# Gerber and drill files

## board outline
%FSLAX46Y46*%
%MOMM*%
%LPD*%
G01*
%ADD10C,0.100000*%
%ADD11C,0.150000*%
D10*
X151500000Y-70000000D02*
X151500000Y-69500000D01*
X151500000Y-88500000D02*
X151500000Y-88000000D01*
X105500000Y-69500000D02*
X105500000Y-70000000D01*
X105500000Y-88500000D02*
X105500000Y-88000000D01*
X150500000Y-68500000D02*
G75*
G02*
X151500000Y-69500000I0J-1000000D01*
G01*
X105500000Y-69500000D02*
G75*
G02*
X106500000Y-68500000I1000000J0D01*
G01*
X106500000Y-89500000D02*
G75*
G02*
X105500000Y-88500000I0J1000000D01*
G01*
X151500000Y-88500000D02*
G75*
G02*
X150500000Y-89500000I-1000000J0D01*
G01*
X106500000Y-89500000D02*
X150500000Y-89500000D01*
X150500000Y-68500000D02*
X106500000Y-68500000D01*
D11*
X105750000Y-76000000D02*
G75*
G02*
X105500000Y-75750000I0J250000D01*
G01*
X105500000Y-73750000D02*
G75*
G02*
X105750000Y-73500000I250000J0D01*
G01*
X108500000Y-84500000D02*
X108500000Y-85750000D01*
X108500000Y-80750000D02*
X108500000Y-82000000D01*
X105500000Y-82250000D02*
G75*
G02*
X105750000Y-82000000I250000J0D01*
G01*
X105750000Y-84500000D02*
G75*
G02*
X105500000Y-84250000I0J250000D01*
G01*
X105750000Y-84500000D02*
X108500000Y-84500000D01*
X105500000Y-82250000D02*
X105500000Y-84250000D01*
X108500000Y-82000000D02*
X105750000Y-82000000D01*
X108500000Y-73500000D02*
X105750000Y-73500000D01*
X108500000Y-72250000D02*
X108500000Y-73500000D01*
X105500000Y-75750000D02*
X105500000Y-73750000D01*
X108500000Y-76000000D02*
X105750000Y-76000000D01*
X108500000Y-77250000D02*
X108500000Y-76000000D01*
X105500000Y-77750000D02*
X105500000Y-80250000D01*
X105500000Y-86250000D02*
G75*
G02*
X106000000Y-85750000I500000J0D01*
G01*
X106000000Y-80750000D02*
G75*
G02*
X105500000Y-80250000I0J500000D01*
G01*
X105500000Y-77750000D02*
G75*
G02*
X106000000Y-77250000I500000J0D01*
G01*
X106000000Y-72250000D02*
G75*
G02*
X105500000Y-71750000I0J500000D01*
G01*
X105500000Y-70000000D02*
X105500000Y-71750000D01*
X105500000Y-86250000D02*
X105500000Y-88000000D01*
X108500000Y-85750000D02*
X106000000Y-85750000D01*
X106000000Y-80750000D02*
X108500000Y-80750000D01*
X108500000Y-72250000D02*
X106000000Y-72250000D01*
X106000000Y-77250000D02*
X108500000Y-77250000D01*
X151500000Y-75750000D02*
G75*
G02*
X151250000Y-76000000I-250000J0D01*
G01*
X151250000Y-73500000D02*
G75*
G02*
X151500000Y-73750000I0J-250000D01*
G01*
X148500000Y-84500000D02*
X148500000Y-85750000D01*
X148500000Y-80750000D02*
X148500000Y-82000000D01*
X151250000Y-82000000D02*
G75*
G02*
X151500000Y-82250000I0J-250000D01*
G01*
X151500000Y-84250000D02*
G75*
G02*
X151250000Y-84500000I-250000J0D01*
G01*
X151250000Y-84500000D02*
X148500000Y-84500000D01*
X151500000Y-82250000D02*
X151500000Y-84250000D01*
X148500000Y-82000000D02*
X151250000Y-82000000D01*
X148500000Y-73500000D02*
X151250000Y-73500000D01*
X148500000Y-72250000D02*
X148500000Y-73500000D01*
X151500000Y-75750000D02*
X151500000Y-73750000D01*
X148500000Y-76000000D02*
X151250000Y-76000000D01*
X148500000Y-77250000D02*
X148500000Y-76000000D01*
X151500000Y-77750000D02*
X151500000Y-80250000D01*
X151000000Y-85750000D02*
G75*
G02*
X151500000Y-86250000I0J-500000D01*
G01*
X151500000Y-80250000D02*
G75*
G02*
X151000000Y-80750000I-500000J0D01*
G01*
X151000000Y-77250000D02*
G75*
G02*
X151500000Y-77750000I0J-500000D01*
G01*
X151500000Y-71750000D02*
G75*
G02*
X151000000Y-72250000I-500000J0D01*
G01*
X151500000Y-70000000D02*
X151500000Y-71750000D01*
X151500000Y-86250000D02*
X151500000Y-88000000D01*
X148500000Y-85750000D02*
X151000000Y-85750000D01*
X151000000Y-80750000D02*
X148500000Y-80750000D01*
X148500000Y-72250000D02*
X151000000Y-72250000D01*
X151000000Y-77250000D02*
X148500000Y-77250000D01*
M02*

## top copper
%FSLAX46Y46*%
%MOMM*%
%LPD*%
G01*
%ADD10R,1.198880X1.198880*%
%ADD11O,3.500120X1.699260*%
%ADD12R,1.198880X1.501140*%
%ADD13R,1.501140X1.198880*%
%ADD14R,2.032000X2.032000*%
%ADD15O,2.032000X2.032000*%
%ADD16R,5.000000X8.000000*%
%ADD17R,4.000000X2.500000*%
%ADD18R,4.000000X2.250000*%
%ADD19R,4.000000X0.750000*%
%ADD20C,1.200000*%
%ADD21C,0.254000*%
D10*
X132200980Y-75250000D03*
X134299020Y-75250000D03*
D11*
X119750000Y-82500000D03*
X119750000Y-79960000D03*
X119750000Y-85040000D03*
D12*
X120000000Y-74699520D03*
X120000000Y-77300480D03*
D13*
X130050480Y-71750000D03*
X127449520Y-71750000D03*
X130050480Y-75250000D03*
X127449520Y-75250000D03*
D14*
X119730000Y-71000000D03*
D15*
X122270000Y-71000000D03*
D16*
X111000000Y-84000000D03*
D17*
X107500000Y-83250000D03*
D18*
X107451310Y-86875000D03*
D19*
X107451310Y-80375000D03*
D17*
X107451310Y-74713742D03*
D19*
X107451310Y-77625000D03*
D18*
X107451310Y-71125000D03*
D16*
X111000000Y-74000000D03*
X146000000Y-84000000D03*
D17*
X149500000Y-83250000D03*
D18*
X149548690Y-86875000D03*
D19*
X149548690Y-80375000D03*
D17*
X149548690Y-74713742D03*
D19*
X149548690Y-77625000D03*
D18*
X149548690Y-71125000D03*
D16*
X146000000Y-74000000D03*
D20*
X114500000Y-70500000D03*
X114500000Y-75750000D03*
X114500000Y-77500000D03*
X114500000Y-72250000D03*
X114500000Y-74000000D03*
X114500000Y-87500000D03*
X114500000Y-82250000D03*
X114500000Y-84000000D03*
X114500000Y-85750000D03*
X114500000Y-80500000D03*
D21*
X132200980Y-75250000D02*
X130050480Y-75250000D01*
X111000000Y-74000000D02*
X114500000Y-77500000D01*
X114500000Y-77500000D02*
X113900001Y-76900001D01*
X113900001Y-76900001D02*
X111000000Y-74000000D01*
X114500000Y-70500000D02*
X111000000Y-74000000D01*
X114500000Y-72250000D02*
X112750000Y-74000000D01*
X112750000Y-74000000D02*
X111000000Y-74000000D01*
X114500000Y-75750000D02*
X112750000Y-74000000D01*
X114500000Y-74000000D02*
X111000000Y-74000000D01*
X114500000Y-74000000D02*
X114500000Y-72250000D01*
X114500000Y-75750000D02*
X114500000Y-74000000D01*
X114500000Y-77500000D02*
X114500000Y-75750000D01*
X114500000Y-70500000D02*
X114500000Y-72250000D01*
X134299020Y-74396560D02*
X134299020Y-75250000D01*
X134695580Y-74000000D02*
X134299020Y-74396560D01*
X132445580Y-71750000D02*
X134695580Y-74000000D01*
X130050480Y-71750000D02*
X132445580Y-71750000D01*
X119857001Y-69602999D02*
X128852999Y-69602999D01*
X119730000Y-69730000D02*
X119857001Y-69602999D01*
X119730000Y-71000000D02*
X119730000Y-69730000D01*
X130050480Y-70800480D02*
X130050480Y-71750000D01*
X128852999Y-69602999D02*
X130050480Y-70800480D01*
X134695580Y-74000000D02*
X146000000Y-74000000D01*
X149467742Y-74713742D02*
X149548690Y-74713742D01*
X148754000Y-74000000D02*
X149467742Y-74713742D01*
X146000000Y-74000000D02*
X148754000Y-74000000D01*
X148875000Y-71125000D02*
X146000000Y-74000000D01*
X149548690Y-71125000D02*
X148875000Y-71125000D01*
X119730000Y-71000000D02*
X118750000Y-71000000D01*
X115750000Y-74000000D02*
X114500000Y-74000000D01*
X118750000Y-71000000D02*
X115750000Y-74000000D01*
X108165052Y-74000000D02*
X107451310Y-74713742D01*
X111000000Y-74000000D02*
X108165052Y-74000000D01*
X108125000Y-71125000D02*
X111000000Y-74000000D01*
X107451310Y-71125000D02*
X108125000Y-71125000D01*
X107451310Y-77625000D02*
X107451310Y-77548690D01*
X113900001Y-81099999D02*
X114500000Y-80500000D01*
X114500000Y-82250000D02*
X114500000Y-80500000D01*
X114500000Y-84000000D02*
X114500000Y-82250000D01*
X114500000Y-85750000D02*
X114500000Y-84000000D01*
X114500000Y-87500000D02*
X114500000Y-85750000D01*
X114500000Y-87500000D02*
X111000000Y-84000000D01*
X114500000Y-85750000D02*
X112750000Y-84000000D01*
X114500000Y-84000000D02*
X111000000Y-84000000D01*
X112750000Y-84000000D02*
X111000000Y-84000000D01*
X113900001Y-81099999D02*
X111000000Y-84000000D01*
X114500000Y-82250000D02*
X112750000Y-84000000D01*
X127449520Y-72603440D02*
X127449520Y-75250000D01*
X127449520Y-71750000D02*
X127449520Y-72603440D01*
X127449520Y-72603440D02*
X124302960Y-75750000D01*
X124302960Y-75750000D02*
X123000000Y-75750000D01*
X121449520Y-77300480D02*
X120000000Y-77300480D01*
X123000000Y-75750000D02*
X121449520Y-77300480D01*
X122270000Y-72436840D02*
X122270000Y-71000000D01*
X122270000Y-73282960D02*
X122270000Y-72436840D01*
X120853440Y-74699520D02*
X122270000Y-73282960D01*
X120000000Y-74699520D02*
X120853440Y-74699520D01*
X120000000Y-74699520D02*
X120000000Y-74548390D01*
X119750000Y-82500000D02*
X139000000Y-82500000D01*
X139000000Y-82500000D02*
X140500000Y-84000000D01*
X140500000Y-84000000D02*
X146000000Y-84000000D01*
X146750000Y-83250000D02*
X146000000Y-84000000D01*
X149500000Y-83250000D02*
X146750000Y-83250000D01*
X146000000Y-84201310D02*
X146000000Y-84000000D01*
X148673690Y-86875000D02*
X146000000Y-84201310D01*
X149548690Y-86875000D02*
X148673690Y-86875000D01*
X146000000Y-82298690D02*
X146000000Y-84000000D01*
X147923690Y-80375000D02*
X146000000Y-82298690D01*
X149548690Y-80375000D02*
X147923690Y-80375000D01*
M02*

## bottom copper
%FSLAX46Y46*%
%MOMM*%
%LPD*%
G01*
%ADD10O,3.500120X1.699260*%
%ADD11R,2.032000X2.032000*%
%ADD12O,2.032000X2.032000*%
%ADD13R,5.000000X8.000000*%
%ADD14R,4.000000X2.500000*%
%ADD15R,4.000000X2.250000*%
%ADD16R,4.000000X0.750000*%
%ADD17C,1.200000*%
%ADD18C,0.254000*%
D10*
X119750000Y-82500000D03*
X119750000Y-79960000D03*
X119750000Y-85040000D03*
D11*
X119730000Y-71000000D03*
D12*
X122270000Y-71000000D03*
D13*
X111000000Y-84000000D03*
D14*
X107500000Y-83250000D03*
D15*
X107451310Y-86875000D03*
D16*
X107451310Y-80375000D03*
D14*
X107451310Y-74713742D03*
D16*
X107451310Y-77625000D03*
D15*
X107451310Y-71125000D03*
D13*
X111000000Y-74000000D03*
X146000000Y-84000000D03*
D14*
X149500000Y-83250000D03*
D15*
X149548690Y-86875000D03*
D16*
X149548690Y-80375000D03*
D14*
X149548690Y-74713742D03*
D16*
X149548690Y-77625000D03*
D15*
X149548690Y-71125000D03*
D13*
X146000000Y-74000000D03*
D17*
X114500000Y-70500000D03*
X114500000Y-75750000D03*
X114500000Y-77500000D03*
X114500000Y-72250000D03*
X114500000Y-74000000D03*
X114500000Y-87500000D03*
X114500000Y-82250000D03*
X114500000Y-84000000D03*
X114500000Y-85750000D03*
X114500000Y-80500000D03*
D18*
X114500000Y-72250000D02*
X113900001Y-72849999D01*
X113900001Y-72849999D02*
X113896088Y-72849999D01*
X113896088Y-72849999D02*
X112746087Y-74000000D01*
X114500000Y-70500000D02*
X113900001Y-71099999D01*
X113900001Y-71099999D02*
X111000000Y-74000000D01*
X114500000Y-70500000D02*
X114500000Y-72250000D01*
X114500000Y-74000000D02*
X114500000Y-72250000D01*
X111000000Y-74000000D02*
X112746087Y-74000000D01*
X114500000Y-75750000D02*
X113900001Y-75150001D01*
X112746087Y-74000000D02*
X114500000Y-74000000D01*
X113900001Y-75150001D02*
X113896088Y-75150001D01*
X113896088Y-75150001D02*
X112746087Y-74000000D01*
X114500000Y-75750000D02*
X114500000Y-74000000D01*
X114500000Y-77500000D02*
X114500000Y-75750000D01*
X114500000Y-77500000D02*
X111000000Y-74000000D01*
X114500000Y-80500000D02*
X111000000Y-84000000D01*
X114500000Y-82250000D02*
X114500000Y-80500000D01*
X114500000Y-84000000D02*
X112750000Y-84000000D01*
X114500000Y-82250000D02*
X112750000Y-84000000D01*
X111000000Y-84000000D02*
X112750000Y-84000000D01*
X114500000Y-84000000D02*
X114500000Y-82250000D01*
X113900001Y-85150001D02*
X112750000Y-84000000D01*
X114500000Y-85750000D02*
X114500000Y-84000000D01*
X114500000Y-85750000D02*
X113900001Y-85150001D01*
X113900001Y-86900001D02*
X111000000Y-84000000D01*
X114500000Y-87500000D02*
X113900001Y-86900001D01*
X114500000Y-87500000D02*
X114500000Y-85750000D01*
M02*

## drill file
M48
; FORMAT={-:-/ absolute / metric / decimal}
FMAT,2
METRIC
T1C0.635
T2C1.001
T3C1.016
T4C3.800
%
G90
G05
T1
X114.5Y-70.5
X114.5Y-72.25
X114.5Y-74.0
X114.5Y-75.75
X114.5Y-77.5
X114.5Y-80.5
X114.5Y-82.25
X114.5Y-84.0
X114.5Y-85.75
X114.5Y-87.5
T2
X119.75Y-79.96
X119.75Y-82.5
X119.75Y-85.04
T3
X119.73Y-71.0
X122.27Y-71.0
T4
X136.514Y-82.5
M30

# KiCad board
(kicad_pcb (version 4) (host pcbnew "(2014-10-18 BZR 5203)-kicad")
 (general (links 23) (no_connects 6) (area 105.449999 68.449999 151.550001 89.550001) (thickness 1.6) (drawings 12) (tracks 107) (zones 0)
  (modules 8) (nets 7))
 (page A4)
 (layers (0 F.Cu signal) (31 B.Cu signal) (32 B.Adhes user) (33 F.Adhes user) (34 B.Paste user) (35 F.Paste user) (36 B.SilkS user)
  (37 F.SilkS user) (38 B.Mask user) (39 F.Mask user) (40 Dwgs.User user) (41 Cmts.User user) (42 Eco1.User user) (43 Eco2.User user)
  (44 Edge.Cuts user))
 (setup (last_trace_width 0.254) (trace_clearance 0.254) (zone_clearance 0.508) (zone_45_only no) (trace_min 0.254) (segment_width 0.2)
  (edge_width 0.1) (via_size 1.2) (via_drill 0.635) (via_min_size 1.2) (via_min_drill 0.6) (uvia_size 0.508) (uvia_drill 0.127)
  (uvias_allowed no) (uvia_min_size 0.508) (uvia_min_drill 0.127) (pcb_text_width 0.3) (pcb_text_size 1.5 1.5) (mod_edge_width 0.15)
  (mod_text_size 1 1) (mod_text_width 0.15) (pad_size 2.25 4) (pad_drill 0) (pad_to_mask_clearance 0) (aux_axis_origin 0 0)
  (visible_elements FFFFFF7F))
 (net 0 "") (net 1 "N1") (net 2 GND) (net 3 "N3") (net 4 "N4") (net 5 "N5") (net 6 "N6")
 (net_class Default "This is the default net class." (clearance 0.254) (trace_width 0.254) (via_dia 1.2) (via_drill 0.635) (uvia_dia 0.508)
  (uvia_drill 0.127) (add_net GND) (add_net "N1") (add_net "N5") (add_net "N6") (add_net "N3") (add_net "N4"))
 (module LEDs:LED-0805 (layer F.Cu) (at 133.25 75.25)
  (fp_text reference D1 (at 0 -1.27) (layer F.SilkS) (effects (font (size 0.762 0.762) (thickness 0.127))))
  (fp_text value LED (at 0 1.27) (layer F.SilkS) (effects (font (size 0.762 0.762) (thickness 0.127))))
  (pad 1 smd rect (at -1.04902 0) (size 1.19888 1.19888) (layers F.Cu F.Paste F.Mask) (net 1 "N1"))
  (pad 2 smd rect (at 1.04902 0) (size 1.19888 1.19888) (layers F.Cu F.Paste F.Mask) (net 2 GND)))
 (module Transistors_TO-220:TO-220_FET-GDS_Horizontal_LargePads (layer F.Cu) (at 119.75 82.5 270)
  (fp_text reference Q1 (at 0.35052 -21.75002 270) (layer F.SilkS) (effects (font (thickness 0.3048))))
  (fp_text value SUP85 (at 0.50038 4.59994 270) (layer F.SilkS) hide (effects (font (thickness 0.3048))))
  (pad D thru_hole oval (at 0 0) (size 3.50012 1.69926) (drill 1.00076) (layers *.Cu *.Mask F.SilkS) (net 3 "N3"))
  (pad G thru_hole oval (at -2.54 0) (size 3.50012 1.69926) (drill 1.00076) (layers *.Cu *.Mask F.SilkS) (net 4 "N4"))
  (pad S thru_hole oval (at 2.54 0) (size 3.50012 1.69926) (drill 1.00076) (layers *.Cu *.Mask F.SilkS) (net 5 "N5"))
  (pad "" np_thru_hole circle (at 0 -16.764) (size 3.79984 3.79984) (drill 3.79984) (layers *.Cu *.Mask F.SilkS)))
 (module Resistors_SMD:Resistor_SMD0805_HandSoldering (layer F.Cu) (at 120 76 270)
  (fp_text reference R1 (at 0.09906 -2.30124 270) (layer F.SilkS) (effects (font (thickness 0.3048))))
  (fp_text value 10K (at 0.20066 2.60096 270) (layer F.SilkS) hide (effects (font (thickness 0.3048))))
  (pad 1 smd rect (at -1.30048 0 270) (size 1.50114 1.19888) (layers F.Cu F.Paste F.Mask) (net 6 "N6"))
  (pad 2 smd rect (at 1.30048 0 270) (size 1.50114 1.19888) (layers F.Cu F.Paste F.Mask) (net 4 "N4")))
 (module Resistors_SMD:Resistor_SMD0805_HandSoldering (layer F.Cu) (at 128.75 71.75 180)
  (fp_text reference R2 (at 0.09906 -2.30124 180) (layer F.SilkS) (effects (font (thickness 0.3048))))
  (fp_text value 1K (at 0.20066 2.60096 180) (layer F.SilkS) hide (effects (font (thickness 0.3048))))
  (pad 1 smd rect (at -1.30048 0 180) (size 1.50114 1.19888) (layers F.Cu F.Paste F.Mask) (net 2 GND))
  (pad 2 smd rect (at 1.30048 0 180) (size 1.50114 1.19888) (layers F.Cu F.Paste F.Mask) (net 4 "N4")))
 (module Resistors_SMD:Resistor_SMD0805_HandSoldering (layer F.Cu) (at 128.75 75.25 180)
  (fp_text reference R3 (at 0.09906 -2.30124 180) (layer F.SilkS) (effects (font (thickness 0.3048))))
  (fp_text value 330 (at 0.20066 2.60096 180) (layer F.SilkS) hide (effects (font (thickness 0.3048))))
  (pad 1 smd rect (at -1.30048 0 180) (size 1.50114 1.19888) (layers F.Cu F.Paste F.Mask) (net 1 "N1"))
  (pad 2 smd rect (at 1.30048 0 180) (size 1.50114 1.19888) (layers F.Cu F.Paste F.Mask) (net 4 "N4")))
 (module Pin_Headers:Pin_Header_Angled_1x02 (layer F.Cu) (at 121 71)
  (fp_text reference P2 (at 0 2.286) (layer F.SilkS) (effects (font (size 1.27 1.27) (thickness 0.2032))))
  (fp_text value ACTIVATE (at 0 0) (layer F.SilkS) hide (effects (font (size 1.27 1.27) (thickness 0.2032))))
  (pad 1 thru_hole rect (at -1.27 0) (size 2.032 2.032) (drill 1.016) (layers *.Cu *.Mask F.SilkS) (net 2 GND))
  (pad 2 thru_hole oval (at 1.27 0) (size 2.032 2.032) (drill 1.016) (layers *.Cu *.Mask F.SilkS) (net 6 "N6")))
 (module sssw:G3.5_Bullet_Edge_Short (layer B.Cu) (at 106 79 270)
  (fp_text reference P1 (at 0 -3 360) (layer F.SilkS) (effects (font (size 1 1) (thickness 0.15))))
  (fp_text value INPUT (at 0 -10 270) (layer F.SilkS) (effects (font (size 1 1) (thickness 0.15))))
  (fp_arc (start -3.25 0.25) (end -3.25 0.5) (angle -90) (layer Edge.Cuts) (width 0.15))
  (fp_arc (start -5.25 0.25) (end -5.5 0.25) (angle -90) (layer Edge.Cuts) (width 0.15))
  (fp_line (start 5.5 -2.5) (end 6.75 -2.5) (layer Edge.Cuts) (width 0.15))
  (fp_line (start 1.75 -2.5) (end 3 -2.5) (layer Edge.Cuts) (width 0.15))
  (fp_arc (start 3.25 0.25) (end 3 0.25) (angle -90) (layer Edge.Cuts) (width 0.15))
  (fp_arc (start 5.25 0.25) (end 5.25 0.5) (angle -90) (layer Edge.Cuts) (width 0.15))
  (fp_line (start 5.5 0.25) (end 5.5 -2.5) (layer Edge.Cuts) (width 0.15))
  (fp_line (start 3.25 0.5) (end 5.25 0.5) (layer Edge.Cuts) (width 0.15))
  (fp_line (start 3 -2.5) (end 3 0.25) (layer Edge.Cuts) (width 0.15))
  (fp_line (start -5.5 -2.5) (end -5.5 0.25) (layer Edge.Cuts) (width 0.15))
  (fp_line (start -6.75 -2.5) (end -5.5 -2.5) (layer Edge.Cuts) (width 0.15))
  (fp_line (start -3.25 0.5) (end -5.25 0.5) (layer Edge.Cuts) (width 0.15))
  (fp_line (start -3 -2.5) (end -3 0.25) (layer Edge.Cuts) (width 0.15))
  (fp_line (start -1.75 -2.5) (end -3 -2.5) (layer Edge.Cuts) (width 0.15))
  (fp_line (start -1.25 0.5) (end 1.25 0.5) (layer Edge.Cuts) (width 0.15))
  (fp_arc (start 7.25 0) (end 6.75 0) (angle -90) (layer Edge.Cuts) (width 0.15))
  (fp_arc (start 1.25 0) (end 1.25 0.5) (angle -90) (layer Edge.Cuts) (width 0.15))
  (fp_arc (start -1.25 0) (end -1.75 0) (angle -90) (layer Edge.Cuts) (width 0.15))
  (fp_arc (start -7.25 0) (end -7.25 0.5) (angle -90) (layer Edge.Cuts) (width 0.15))
  (fp_line (start -9 0.5) (end -7.25 0.5) (layer Edge.Cuts) (width 0.15))
  (fp_line (start 7.25 0.5) (end 9 0.5) (layer Edge.Cuts) (width 0.15))
  (fp_line (start 6.75 -2.5) (end 6.75 0) (layer Edge.Cuts) (width 0.15))
  (fp_line (start 1.75 0) (end 1.75 -2.5) (layer Edge.Cuts) (width 0.15))
  (fp_line (start -6.75 -2.5) (end -6.75 0) (layer Edge.Cuts) (width 0.15))
  (fp_line (start -1.75 0) (end -1.75 -2.5) (layer Edge.Cuts) (width 0.15))
  (pad 2 connect rect (at 5 -5 270) (size 8 5) (layers *.Cu *.Mask) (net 5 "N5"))
  (pad 2 smd rect (at 4.25 -1.5 270) (size 2.5 4) (layers *.Cu *.Mask) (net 5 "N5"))
  (pad 2 smd rect (at 7.875 -1.45131 270) (size 2.25 4) (layers *.Cu *.Mask) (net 5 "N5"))
  (pad 2 smd rect (at 1.375 -1.45131 270) (size 0.75 4) (layers *.Cu *.Mask) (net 5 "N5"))
  (pad 1 smd rect (at -4.286258 -1.45131 90) (size 2.5 4) (layers *.Cu *.Mask) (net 2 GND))
  (pad 1 smd rect (at -1.375 -1.45131 90) (size 0.75 4) (layers *.Cu *.Mask) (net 2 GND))
  (pad 1 smd rect (at -7.875 -1.45131 90) (size 2.25 4) (layers *.Cu *.Mask) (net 2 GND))
  (pad 1 connect rect (at -5 -5 90) (size 8 5) (layers *.Cu *.Mask) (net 2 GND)))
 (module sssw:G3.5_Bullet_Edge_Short (layer F.Cu) (at 151 79 270)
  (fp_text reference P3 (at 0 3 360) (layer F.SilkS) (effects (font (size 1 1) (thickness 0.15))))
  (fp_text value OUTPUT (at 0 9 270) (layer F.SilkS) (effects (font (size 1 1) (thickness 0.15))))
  (fp_arc (start -3.25 -0.25) (end -3.25 -0.5) (angle 90) (layer Edge.Cuts) (width 0.15))
  (fp_arc (start -5.25 -0.25) (end -5.5 -0.25) (angle 90) (layer Edge.Cuts) (width 0.15))
  (fp_line (start 5.5 2.5) (end 6.75 2.5) (layer Edge.Cuts) (width 0.15))
  (fp_line (start 1.75 2.5) (end 3 2.5) (layer Edge.Cuts) (width 0.15))
  (fp_arc (start 3.25 -0.25) (end 3 -0.25) (angle 90) (layer Edge.Cuts) (width 0.15))
  (fp_arc (start 5.25 -0.25) (end 5.25 -0.5) (angle 90) (layer Edge.Cuts) (width 0.15))
  (fp_line (start 5.5 -0.25) (end 5.5 2.5) (layer Edge.Cuts) (width 0.15))
  (fp_line (start 3.25 -0.5) (end 5.25 -0.5) (layer Edge.Cuts) (width 0.15))
  (fp_line (start 3 2.5) (end 3 -0.25) (layer Edge.Cuts) (width 0.15))
  (fp_line (start -5.5 2.5) (end -5.5 -0.25) (layer Edge.Cuts) (width 0.15))
  (fp_line (start -6.75 2.5) (end -5.5 2.5) (layer Edge.Cuts) (width 0.15))
  (fp_line (start -3.25 -0.5) (end -5.25 -0.5) (layer Edge.Cuts) (width 0.15))
  (fp_line (start -3 2.5) (end -3 -0.25) (layer Edge.Cuts) (width 0.15))
  (fp_line (start -1.75 2.5) (end -3 2.5) (layer Edge.Cuts) (width 0.15))
  (fp_line (start -1.25 -0.5) (end 1.25 -0.5) (layer Edge.Cuts) (width 0.15))
  (fp_arc (start 7.25 0) (end 6.75 0) (angle 90) (layer Edge.Cuts) (width 0.15))
  (fp_arc (start 1.25 0) (end 1.25 -0.5) (angle 90) (layer Edge.Cuts) (width 0.15))
  (fp_arc (start -1.25 0) (end -1.75 0) (angle 90) (layer Edge.Cuts) (width 0.15))
  (fp_arc (start -7.25 0) (end -7.25 -0.5) (angle 90) (layer Edge.Cuts) (width 0.15))
  (fp_line (start -9 -0.5) (end -7.25 -0.5) (layer Edge.Cuts) (width 0.15))
  (fp_line (start 7.25 -0.5) (end 9 -0.5) (layer Edge.Cuts) (width 0.15))
  (fp_line (start 6.75 2.5) (end 6.75 0) (layer Edge.Cuts) (width 0.15))
  (fp_line (start 1.75 0) (end 1.75 2.5) (layer Edge.Cuts) (width 0.15))
  (fp_line (start -6.75 2.5) (end -6.75 0) (layer Edge.Cuts) (width 0.15))
  (fp_line (start -1.75 0) (end -1.75 2.5) (layer Edge.Cuts) (width 0.15))
  (pad 2 connect rect (at 5 5 270) (size 8 5) (layers *.Cu *.Mask) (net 3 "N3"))
  (pad 2 smd rect (at 4.25 1.5 270) (size 2.5 4) (layers *.Cu *.Mask) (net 3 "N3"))
  (pad 2 smd rect (at 7.875 1.45131 270) (size 2.25 4) (layers *.Cu *.Mask) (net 3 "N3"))
  (pad 2 smd rect (at 1.375 1.45131 270) (size 0.75 4) (layers *.Cu *.Mask) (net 3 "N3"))
  (pad 1 smd rect (at -4.286258 1.45131 90) (size 2.5 4) (layers *.Cu *.Mask) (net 2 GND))
  (pad 1 smd rect (at -1.375 1.45131 90) (size 0.75 4) (layers *.Cu *.Mask) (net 2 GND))
  (pad 1 smd rect (at -7.875 1.45131 90) (size 2.25 4) (layers *.Cu *.Mask) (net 2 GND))
  (pad 1 connect rect (at -5 5 90) (size 8 5) (layers *.Cu *.Mask) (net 2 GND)))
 (gr_line (start 151.5 70) (end 151.5 69.5) (layer Edge.Cuts) (width 0.1))
 (gr_line (start 151.5 88.5) (end 151.5 88) (layer Edge.Cuts) (width 0.1))
 (gr_line (start 105.5 69.5) (end 105.5 70) (layer Edge.Cuts) (width 0.1))
 (gr_line (start 105.5 88.5) (end 105.5 88) (layer Edge.Cuts) (width 0.1))
 (gr_arc (start 150.5 69.5) (end 151.5 69.5) (angle -90) (layer Edge.Cuts) (width 0.1))
 (gr_arc (start 106.5 69.5) (end 106.5 68.5) (angle -90) (layer Edge.Cuts) (width 0.1))
 (gr_arc (start 106.5 88.5) (end 105.5 88.5) (angle -90) (layer Edge.Cuts) (width 0.1))
 (gr_arc (start 150.5 88.5) (end 151.5 88.5) (angle 90) (layer Edge.Cuts) (width 0.1))
 (gr_line (start 106.5 89.5) (end 150.5 89.5) (layer Edge.Cuts) (width 0.1))
 (gr_line (start 150.5 68.5) (end 106.5 68.5) (layer Edge.Cuts) (width 0.1))
 (segment (start 119.75 79.96) (end 119.75 80) (width 0.254) (layer Edge.Cuts) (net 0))
 (segment (start 132.20098 75.25) (end 130.05048 75.25) (width 0.254) (layer F.Cu) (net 1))
 (segment (start 114.5 72.25) (end 113.900001 72.849999) (width 0.254) (layer B.Cu) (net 2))
 (segment (start 113.900001 72.849999) (end 113.896088 72.849999) (width 0.254) (layer B.Cu) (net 2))
 (segment (start 113.896088 72.849999) (end 112.746087 74) (width 0.254) (layer B.Cu) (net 2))
 (segment (start 114.5 70.5) (end 113.900001 71.099999) (width 0.254) (layer B.Cu) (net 2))
 (segment (start 113.900001 71.099999) (end 111 74) (width 0.254) (layer B.Cu) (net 2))
 (segment (start 114.5 70.5) (end 114.5 72.25) (width 0.254) (layer B.Cu) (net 2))
 (segment (start 114.5 74) (end 114.5 72.25) (width 0.254) (layer B.Cu) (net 2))
 (segment (start 111 74) (end 112.746087 74) (width 0.254) (layer B.Cu) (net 2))
 (segment (start 114.5 75.75) (end 113.900001 75.150001) (width 0.254) (layer B.Cu) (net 2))
 (segment (start 112.746087 74) (end 114.5 74) (width 0.254) (layer B.Cu) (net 2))
 (segment (start 113.900001 75.150001) (end 113.896088 75.150001) (width 0.254) (layer B.Cu) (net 2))
 (segment (start 113.896088 75.150001) (end 112.746087 74) (width 0.254) (layer B.Cu) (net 2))
 (segment (start 114.5 75.75) (end 114.5 74) (width 0.254) (layer B.Cu) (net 2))
 (segment (start 114.5 77.5) (end 114.5 75.75) (width 0.254) (layer B.Cu) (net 2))
 (segment (start 114.5 77.5) (end 111 74) (width 0.254) (layer B.Cu) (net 2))
 (segment (start 111 74) (end 114.5 77.5) (width 0.254) (layer F.Cu) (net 2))
 (segment (start 114.5 77.5) (end 113.900001 76.900001) (width 0.254) (layer F.Cu) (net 2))
 (segment (start 113.900001 76.900001) (end 111 74) (width 0.254) (layer F.Cu) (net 2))
 (segment (start 114.5 70.5) (end 111 74) (width 0.254) (layer F.Cu) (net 2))
 (segment (start 114.5 72.25) (end 112.75 74) (width 0.254) (layer F.Cu) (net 2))
 (segment (start 112.75 74) (end 111 74) (width 0.254) (layer F.Cu) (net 2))
 (segment (start 114.5 75.75) (end 112.75 74) (width 0.254) (layer F.Cu) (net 2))
 (segment (start 114.5 74) (end 111 74) (width 0.254) (layer F.Cu) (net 2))
 (segment (start 114.5 74) (end 114.5 72.25) (width 0.254) (layer F.Cu) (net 2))
 (segment (start 114.5 75.75) (end 114.5 74) (width 0.254) (layer F.Cu) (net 2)) (via (at 114.5 70.5) (size 1.2) (layers F.Cu B.Cu) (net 2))
 (via (at 114.5 75.75) (size 1.2) (layers F.Cu B.Cu) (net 2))
 (segment (start 114.5 77.5) (end 114.5 75.75) (width 0.254) (layer F.Cu) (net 2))
 (via (at 114.5 77.5) (size 1.2) (layers F.Cu B.Cu) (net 2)) (via (at 114.5 72.25) (size 1.2) (layers F.Cu B.Cu) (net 2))
 (segment (start 114.5 70.5) (end 114.5 72.25) (width 0.254) (layer F.Cu) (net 2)) (via (at 114.5 74) (size 1.2) (layers F.Cu B.Cu) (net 2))
 (segment (start 134.29902 74.39656) (end 134.29902 75.25) (width 0.254) (layer F.Cu) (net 2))
 (segment (start 134.69558 74) (end 134.29902 74.39656) (width 0.254) (layer F.Cu) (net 2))
 (segment (start 132.44558 71.75) (end 134.69558 74) (width 0.254) (layer F.Cu) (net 2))
 (segment (start 130.05048 71.75) (end 132.44558 71.75) (width 0.254) (layer F.Cu) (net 2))
 (segment (start 119.857001 69.602999) (end 128.852999 69.602999) (width 0.254) (layer F.Cu) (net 2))
 (segment (start 119.73 69.73) (end 119.857001 69.602999) (width 0.254) (layer F.Cu) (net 2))
 (segment (start 119.73 71) (end 119.73 69.73) (width 0.254) (layer F.Cu) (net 2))
 (segment (start 130.05048 70.80048) (end 130.05048 71.75) (width 0.254) (layer F.Cu) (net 2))
 (segment (start 128.852999 69.602999) (end 130.05048 70.80048) (width 0.254) (layer F.Cu) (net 2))
 (segment (start 134.69558 74) (end 146 74) (width 0.254) (layer F.Cu) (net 2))
 (segment (start 149.467742 74.713742) (end 149.54869 74.713742) (width 0.254) (layer F.Cu) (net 2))
 (segment (start 148.754 74) (end 149.467742 74.713742) (width 0.254) (layer F.Cu) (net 2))
 (segment (start 146 74) (end 148.754 74) (width 0.254) (layer F.Cu) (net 2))
 (segment (start 148.875 71.125) (end 146 74) (width 0.254) (layer F.Cu) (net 2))
 (segment (start 149.54869 71.125) (end 148.875 71.125) (width 0.254) (layer F.Cu) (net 2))
 (segment (start 119.73 71) (end 118.75 71) (width 0.254) (layer F.Cu) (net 2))
 (segment (start 115.75 74) (end 114.5 74) (width 0.254) (layer F.Cu) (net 2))
 (segment (start 118.75 71) (end 115.75 74) (width 0.254) (layer F.Cu) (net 2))
 (segment (start 108.165052 74) (end 107.45131 74.713742) (width 0.254) (layer F.Cu) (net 2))
 (segment (start 111 74) (end 108.165052 74) (width 0.254) (layer F.Cu) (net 2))
 (segment (start 108.125 71.125) (end 111 74) (width 0.254) (layer F.Cu) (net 2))
 (segment (start 107.45131 71.125) (end 108.125 71.125) (width 0.254) (layer F.Cu) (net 2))
 (segment (start 107.45131 77.625) (end 107.45131 77.54869) (width 0.254) (layer F.Cu) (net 2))
 (segment (start 113.900001 81.099999) (end 114.5 80.5) (width 0.254) (layer F.Cu) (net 5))
 (segment (start 114.5 82.25) (end 114.5 80.5) (width 0.254) (layer F.Cu) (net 5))
 (segment (start 114.5 84) (end 114.5 82.25) (width 0.254) (layer F.Cu) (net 5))
 (segment (start 114.5 85.75) (end 114.5 84) (width 0.254) (layer F.Cu) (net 5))
 (segment (start 114.5 87.5) (end 114.5 85.75) (width 0.254) (layer F.Cu) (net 5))
 (segment (start 114.5 87.5) (end 111 84) (width 0.254) (layer F.Cu) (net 5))
 (segment (start 114.5 85.75) (end 112.75 84) (width 0.254) (layer F.Cu) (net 5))
 (via (at 114.5 87.5) (size 1.2) (layers F.Cu B.Cu) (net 5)) (via (at 114.5 82.25) (size 1.2) (layers F.Cu B.Cu) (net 5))
 (via (at 114.5 84) (size 1.2) (layers F.Cu B.Cu) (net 5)) (via (at 114.5 85.75) (size 1.2) (layers F.Cu B.Cu) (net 5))
 (segment (start 114.5 84) (end 111 84) (width 0.254) (layer F.Cu) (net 5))
 (segment (start 112.75 84) (end 111 84) (width 0.254) (layer F.Cu) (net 5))
 (segment (start 113.900001 81.099999) (end 111 84) (width 0.254) (layer F.Cu) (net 5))
 (segment (start 114.5 82.25) (end 112.75 84) (width 0.254) (layer F.Cu) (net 5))
 (via (at 114.5 80.5) (size 1.2) (layers F.Cu B.Cu) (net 5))
 (segment (start 114.5 80.5) (end 111 84) (width 0.254) (layer B.Cu) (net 5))
 (segment (start 114.5 82.25) (end 114.5 80.5) (width 0.254) (layer B.Cu) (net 5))
 (segment (start 114.5 84) (end 112.75 84) (width 0.254) (layer B.Cu) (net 5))
 (segment (start 114.5 82.25) (end 112.75 84) (width 0.254) (layer B.Cu) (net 5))
 (segment (start 111 84) (end 112.75 84) (width 0.254) (layer B.Cu) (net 5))
 (segment (start 114.5 84) (end 114.5 82.25) (width 0.254) (layer B.Cu) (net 5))
 (segment (start 113.900001 85.150001) (end 112.75 84) (width 0.254) (layer B.Cu) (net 5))
 (segment (start 114.5 85.75) (end 114.5 84) (width 0.254) (layer B.Cu) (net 5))
 (segment (start 114.5 85.75) (end 113.900001 85.150001) (width 0.254) (layer B.Cu) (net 5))
 (segment (start 113.900001 86.900001) (end 111 84) (width 0.254) (layer B.Cu) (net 5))
 (segment (start 114.5 87.5) (end 113.900001 86.900001) (width 0.254) (layer B.Cu) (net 5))
 (segment (start 114.5 87.5) (end 114.5 85.75) (width 0.254) (layer B.Cu) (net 5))
 (segment (start 127.44952 72.60344) (end 127.44952 75.25) (width 0.254) (layer F.Cu) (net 4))
 (segment (start 127.44952 71.75) (end 127.44952 72.60344) (width 0.254) (layer F.Cu) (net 4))
 (segment (start 127.44952 72.60344) (end 124.30296 75.75) (width 0.254) (layer F.Cu) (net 4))
 (segment (start 124.30296 75.75) (end 123 75.75) (width 0.254) (layer F.Cu) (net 4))
 (segment (start 121.44952 77.30048) (end 120 77.30048) (width 0.254) (layer F.Cu) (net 4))
 (segment (start 123 75.75) (end 121.44952 77.30048) (width 0.254) (layer F.Cu) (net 4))
 (segment (start 122.27 72.43684) (end 122.27 71) (width 0.254) (layer F.Cu) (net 6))
 (segment (start 122.27 73.28296) (end 122.27 72.43684) (width 0.254) (layer F.Cu) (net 6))
 (segment (start 120.85344 74.69952) (end 122.27 73.28296) (width 0.254) (layer F.Cu) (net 6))
 (segment (start 120 74.69952) (end 120.85344 74.69952) (width 0.254) (layer F.Cu) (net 6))
 (segment (start 120 74.69952) (end 120 74.54839) (width 0.254) (layer F.Cu) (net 6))
 (segment (start 119.75 82.5) (end 139 82.5) (width 0.254) (layer F.Cu) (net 3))
 (segment (start 139 82.5) (end 140.5 84) (width 0.254) (layer F.Cu) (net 3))
 (segment (start 140.5 84) (end 146 84) (width 0.254) (layer F.Cu) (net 3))
 (segment (start 146.75 83.25) (end 146 84) (width 0.254) (layer F.Cu) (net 3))
 (segment (start 149.5 83.25) (end 146.75 83.25) (width 0.254) (layer F.Cu) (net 3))
 (segment (start 146 84.20131) (end 146 84) (width 0.254) (layer F.Cu) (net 3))
 (segment (start 148.67369 86.875) (end 146 84.20131) (width 0.254) (layer F.Cu) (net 3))
 (segment (start 149.54869 86.875) (end 148.67369 86.875) (width 0.254) (layer F.Cu) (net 3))
 (segment (start 146 82.29869) (end 146 84) (width 0.254) (layer F.Cu) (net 3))
 (segment (start 147.92369 80.375) (end 146 82.29869) (width 0.254) (layer F.Cu) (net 3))
 (segment (start 149.54869 80.375) (end 147.92369 80.375) (width 0.254) (layer F.Cu) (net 3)))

